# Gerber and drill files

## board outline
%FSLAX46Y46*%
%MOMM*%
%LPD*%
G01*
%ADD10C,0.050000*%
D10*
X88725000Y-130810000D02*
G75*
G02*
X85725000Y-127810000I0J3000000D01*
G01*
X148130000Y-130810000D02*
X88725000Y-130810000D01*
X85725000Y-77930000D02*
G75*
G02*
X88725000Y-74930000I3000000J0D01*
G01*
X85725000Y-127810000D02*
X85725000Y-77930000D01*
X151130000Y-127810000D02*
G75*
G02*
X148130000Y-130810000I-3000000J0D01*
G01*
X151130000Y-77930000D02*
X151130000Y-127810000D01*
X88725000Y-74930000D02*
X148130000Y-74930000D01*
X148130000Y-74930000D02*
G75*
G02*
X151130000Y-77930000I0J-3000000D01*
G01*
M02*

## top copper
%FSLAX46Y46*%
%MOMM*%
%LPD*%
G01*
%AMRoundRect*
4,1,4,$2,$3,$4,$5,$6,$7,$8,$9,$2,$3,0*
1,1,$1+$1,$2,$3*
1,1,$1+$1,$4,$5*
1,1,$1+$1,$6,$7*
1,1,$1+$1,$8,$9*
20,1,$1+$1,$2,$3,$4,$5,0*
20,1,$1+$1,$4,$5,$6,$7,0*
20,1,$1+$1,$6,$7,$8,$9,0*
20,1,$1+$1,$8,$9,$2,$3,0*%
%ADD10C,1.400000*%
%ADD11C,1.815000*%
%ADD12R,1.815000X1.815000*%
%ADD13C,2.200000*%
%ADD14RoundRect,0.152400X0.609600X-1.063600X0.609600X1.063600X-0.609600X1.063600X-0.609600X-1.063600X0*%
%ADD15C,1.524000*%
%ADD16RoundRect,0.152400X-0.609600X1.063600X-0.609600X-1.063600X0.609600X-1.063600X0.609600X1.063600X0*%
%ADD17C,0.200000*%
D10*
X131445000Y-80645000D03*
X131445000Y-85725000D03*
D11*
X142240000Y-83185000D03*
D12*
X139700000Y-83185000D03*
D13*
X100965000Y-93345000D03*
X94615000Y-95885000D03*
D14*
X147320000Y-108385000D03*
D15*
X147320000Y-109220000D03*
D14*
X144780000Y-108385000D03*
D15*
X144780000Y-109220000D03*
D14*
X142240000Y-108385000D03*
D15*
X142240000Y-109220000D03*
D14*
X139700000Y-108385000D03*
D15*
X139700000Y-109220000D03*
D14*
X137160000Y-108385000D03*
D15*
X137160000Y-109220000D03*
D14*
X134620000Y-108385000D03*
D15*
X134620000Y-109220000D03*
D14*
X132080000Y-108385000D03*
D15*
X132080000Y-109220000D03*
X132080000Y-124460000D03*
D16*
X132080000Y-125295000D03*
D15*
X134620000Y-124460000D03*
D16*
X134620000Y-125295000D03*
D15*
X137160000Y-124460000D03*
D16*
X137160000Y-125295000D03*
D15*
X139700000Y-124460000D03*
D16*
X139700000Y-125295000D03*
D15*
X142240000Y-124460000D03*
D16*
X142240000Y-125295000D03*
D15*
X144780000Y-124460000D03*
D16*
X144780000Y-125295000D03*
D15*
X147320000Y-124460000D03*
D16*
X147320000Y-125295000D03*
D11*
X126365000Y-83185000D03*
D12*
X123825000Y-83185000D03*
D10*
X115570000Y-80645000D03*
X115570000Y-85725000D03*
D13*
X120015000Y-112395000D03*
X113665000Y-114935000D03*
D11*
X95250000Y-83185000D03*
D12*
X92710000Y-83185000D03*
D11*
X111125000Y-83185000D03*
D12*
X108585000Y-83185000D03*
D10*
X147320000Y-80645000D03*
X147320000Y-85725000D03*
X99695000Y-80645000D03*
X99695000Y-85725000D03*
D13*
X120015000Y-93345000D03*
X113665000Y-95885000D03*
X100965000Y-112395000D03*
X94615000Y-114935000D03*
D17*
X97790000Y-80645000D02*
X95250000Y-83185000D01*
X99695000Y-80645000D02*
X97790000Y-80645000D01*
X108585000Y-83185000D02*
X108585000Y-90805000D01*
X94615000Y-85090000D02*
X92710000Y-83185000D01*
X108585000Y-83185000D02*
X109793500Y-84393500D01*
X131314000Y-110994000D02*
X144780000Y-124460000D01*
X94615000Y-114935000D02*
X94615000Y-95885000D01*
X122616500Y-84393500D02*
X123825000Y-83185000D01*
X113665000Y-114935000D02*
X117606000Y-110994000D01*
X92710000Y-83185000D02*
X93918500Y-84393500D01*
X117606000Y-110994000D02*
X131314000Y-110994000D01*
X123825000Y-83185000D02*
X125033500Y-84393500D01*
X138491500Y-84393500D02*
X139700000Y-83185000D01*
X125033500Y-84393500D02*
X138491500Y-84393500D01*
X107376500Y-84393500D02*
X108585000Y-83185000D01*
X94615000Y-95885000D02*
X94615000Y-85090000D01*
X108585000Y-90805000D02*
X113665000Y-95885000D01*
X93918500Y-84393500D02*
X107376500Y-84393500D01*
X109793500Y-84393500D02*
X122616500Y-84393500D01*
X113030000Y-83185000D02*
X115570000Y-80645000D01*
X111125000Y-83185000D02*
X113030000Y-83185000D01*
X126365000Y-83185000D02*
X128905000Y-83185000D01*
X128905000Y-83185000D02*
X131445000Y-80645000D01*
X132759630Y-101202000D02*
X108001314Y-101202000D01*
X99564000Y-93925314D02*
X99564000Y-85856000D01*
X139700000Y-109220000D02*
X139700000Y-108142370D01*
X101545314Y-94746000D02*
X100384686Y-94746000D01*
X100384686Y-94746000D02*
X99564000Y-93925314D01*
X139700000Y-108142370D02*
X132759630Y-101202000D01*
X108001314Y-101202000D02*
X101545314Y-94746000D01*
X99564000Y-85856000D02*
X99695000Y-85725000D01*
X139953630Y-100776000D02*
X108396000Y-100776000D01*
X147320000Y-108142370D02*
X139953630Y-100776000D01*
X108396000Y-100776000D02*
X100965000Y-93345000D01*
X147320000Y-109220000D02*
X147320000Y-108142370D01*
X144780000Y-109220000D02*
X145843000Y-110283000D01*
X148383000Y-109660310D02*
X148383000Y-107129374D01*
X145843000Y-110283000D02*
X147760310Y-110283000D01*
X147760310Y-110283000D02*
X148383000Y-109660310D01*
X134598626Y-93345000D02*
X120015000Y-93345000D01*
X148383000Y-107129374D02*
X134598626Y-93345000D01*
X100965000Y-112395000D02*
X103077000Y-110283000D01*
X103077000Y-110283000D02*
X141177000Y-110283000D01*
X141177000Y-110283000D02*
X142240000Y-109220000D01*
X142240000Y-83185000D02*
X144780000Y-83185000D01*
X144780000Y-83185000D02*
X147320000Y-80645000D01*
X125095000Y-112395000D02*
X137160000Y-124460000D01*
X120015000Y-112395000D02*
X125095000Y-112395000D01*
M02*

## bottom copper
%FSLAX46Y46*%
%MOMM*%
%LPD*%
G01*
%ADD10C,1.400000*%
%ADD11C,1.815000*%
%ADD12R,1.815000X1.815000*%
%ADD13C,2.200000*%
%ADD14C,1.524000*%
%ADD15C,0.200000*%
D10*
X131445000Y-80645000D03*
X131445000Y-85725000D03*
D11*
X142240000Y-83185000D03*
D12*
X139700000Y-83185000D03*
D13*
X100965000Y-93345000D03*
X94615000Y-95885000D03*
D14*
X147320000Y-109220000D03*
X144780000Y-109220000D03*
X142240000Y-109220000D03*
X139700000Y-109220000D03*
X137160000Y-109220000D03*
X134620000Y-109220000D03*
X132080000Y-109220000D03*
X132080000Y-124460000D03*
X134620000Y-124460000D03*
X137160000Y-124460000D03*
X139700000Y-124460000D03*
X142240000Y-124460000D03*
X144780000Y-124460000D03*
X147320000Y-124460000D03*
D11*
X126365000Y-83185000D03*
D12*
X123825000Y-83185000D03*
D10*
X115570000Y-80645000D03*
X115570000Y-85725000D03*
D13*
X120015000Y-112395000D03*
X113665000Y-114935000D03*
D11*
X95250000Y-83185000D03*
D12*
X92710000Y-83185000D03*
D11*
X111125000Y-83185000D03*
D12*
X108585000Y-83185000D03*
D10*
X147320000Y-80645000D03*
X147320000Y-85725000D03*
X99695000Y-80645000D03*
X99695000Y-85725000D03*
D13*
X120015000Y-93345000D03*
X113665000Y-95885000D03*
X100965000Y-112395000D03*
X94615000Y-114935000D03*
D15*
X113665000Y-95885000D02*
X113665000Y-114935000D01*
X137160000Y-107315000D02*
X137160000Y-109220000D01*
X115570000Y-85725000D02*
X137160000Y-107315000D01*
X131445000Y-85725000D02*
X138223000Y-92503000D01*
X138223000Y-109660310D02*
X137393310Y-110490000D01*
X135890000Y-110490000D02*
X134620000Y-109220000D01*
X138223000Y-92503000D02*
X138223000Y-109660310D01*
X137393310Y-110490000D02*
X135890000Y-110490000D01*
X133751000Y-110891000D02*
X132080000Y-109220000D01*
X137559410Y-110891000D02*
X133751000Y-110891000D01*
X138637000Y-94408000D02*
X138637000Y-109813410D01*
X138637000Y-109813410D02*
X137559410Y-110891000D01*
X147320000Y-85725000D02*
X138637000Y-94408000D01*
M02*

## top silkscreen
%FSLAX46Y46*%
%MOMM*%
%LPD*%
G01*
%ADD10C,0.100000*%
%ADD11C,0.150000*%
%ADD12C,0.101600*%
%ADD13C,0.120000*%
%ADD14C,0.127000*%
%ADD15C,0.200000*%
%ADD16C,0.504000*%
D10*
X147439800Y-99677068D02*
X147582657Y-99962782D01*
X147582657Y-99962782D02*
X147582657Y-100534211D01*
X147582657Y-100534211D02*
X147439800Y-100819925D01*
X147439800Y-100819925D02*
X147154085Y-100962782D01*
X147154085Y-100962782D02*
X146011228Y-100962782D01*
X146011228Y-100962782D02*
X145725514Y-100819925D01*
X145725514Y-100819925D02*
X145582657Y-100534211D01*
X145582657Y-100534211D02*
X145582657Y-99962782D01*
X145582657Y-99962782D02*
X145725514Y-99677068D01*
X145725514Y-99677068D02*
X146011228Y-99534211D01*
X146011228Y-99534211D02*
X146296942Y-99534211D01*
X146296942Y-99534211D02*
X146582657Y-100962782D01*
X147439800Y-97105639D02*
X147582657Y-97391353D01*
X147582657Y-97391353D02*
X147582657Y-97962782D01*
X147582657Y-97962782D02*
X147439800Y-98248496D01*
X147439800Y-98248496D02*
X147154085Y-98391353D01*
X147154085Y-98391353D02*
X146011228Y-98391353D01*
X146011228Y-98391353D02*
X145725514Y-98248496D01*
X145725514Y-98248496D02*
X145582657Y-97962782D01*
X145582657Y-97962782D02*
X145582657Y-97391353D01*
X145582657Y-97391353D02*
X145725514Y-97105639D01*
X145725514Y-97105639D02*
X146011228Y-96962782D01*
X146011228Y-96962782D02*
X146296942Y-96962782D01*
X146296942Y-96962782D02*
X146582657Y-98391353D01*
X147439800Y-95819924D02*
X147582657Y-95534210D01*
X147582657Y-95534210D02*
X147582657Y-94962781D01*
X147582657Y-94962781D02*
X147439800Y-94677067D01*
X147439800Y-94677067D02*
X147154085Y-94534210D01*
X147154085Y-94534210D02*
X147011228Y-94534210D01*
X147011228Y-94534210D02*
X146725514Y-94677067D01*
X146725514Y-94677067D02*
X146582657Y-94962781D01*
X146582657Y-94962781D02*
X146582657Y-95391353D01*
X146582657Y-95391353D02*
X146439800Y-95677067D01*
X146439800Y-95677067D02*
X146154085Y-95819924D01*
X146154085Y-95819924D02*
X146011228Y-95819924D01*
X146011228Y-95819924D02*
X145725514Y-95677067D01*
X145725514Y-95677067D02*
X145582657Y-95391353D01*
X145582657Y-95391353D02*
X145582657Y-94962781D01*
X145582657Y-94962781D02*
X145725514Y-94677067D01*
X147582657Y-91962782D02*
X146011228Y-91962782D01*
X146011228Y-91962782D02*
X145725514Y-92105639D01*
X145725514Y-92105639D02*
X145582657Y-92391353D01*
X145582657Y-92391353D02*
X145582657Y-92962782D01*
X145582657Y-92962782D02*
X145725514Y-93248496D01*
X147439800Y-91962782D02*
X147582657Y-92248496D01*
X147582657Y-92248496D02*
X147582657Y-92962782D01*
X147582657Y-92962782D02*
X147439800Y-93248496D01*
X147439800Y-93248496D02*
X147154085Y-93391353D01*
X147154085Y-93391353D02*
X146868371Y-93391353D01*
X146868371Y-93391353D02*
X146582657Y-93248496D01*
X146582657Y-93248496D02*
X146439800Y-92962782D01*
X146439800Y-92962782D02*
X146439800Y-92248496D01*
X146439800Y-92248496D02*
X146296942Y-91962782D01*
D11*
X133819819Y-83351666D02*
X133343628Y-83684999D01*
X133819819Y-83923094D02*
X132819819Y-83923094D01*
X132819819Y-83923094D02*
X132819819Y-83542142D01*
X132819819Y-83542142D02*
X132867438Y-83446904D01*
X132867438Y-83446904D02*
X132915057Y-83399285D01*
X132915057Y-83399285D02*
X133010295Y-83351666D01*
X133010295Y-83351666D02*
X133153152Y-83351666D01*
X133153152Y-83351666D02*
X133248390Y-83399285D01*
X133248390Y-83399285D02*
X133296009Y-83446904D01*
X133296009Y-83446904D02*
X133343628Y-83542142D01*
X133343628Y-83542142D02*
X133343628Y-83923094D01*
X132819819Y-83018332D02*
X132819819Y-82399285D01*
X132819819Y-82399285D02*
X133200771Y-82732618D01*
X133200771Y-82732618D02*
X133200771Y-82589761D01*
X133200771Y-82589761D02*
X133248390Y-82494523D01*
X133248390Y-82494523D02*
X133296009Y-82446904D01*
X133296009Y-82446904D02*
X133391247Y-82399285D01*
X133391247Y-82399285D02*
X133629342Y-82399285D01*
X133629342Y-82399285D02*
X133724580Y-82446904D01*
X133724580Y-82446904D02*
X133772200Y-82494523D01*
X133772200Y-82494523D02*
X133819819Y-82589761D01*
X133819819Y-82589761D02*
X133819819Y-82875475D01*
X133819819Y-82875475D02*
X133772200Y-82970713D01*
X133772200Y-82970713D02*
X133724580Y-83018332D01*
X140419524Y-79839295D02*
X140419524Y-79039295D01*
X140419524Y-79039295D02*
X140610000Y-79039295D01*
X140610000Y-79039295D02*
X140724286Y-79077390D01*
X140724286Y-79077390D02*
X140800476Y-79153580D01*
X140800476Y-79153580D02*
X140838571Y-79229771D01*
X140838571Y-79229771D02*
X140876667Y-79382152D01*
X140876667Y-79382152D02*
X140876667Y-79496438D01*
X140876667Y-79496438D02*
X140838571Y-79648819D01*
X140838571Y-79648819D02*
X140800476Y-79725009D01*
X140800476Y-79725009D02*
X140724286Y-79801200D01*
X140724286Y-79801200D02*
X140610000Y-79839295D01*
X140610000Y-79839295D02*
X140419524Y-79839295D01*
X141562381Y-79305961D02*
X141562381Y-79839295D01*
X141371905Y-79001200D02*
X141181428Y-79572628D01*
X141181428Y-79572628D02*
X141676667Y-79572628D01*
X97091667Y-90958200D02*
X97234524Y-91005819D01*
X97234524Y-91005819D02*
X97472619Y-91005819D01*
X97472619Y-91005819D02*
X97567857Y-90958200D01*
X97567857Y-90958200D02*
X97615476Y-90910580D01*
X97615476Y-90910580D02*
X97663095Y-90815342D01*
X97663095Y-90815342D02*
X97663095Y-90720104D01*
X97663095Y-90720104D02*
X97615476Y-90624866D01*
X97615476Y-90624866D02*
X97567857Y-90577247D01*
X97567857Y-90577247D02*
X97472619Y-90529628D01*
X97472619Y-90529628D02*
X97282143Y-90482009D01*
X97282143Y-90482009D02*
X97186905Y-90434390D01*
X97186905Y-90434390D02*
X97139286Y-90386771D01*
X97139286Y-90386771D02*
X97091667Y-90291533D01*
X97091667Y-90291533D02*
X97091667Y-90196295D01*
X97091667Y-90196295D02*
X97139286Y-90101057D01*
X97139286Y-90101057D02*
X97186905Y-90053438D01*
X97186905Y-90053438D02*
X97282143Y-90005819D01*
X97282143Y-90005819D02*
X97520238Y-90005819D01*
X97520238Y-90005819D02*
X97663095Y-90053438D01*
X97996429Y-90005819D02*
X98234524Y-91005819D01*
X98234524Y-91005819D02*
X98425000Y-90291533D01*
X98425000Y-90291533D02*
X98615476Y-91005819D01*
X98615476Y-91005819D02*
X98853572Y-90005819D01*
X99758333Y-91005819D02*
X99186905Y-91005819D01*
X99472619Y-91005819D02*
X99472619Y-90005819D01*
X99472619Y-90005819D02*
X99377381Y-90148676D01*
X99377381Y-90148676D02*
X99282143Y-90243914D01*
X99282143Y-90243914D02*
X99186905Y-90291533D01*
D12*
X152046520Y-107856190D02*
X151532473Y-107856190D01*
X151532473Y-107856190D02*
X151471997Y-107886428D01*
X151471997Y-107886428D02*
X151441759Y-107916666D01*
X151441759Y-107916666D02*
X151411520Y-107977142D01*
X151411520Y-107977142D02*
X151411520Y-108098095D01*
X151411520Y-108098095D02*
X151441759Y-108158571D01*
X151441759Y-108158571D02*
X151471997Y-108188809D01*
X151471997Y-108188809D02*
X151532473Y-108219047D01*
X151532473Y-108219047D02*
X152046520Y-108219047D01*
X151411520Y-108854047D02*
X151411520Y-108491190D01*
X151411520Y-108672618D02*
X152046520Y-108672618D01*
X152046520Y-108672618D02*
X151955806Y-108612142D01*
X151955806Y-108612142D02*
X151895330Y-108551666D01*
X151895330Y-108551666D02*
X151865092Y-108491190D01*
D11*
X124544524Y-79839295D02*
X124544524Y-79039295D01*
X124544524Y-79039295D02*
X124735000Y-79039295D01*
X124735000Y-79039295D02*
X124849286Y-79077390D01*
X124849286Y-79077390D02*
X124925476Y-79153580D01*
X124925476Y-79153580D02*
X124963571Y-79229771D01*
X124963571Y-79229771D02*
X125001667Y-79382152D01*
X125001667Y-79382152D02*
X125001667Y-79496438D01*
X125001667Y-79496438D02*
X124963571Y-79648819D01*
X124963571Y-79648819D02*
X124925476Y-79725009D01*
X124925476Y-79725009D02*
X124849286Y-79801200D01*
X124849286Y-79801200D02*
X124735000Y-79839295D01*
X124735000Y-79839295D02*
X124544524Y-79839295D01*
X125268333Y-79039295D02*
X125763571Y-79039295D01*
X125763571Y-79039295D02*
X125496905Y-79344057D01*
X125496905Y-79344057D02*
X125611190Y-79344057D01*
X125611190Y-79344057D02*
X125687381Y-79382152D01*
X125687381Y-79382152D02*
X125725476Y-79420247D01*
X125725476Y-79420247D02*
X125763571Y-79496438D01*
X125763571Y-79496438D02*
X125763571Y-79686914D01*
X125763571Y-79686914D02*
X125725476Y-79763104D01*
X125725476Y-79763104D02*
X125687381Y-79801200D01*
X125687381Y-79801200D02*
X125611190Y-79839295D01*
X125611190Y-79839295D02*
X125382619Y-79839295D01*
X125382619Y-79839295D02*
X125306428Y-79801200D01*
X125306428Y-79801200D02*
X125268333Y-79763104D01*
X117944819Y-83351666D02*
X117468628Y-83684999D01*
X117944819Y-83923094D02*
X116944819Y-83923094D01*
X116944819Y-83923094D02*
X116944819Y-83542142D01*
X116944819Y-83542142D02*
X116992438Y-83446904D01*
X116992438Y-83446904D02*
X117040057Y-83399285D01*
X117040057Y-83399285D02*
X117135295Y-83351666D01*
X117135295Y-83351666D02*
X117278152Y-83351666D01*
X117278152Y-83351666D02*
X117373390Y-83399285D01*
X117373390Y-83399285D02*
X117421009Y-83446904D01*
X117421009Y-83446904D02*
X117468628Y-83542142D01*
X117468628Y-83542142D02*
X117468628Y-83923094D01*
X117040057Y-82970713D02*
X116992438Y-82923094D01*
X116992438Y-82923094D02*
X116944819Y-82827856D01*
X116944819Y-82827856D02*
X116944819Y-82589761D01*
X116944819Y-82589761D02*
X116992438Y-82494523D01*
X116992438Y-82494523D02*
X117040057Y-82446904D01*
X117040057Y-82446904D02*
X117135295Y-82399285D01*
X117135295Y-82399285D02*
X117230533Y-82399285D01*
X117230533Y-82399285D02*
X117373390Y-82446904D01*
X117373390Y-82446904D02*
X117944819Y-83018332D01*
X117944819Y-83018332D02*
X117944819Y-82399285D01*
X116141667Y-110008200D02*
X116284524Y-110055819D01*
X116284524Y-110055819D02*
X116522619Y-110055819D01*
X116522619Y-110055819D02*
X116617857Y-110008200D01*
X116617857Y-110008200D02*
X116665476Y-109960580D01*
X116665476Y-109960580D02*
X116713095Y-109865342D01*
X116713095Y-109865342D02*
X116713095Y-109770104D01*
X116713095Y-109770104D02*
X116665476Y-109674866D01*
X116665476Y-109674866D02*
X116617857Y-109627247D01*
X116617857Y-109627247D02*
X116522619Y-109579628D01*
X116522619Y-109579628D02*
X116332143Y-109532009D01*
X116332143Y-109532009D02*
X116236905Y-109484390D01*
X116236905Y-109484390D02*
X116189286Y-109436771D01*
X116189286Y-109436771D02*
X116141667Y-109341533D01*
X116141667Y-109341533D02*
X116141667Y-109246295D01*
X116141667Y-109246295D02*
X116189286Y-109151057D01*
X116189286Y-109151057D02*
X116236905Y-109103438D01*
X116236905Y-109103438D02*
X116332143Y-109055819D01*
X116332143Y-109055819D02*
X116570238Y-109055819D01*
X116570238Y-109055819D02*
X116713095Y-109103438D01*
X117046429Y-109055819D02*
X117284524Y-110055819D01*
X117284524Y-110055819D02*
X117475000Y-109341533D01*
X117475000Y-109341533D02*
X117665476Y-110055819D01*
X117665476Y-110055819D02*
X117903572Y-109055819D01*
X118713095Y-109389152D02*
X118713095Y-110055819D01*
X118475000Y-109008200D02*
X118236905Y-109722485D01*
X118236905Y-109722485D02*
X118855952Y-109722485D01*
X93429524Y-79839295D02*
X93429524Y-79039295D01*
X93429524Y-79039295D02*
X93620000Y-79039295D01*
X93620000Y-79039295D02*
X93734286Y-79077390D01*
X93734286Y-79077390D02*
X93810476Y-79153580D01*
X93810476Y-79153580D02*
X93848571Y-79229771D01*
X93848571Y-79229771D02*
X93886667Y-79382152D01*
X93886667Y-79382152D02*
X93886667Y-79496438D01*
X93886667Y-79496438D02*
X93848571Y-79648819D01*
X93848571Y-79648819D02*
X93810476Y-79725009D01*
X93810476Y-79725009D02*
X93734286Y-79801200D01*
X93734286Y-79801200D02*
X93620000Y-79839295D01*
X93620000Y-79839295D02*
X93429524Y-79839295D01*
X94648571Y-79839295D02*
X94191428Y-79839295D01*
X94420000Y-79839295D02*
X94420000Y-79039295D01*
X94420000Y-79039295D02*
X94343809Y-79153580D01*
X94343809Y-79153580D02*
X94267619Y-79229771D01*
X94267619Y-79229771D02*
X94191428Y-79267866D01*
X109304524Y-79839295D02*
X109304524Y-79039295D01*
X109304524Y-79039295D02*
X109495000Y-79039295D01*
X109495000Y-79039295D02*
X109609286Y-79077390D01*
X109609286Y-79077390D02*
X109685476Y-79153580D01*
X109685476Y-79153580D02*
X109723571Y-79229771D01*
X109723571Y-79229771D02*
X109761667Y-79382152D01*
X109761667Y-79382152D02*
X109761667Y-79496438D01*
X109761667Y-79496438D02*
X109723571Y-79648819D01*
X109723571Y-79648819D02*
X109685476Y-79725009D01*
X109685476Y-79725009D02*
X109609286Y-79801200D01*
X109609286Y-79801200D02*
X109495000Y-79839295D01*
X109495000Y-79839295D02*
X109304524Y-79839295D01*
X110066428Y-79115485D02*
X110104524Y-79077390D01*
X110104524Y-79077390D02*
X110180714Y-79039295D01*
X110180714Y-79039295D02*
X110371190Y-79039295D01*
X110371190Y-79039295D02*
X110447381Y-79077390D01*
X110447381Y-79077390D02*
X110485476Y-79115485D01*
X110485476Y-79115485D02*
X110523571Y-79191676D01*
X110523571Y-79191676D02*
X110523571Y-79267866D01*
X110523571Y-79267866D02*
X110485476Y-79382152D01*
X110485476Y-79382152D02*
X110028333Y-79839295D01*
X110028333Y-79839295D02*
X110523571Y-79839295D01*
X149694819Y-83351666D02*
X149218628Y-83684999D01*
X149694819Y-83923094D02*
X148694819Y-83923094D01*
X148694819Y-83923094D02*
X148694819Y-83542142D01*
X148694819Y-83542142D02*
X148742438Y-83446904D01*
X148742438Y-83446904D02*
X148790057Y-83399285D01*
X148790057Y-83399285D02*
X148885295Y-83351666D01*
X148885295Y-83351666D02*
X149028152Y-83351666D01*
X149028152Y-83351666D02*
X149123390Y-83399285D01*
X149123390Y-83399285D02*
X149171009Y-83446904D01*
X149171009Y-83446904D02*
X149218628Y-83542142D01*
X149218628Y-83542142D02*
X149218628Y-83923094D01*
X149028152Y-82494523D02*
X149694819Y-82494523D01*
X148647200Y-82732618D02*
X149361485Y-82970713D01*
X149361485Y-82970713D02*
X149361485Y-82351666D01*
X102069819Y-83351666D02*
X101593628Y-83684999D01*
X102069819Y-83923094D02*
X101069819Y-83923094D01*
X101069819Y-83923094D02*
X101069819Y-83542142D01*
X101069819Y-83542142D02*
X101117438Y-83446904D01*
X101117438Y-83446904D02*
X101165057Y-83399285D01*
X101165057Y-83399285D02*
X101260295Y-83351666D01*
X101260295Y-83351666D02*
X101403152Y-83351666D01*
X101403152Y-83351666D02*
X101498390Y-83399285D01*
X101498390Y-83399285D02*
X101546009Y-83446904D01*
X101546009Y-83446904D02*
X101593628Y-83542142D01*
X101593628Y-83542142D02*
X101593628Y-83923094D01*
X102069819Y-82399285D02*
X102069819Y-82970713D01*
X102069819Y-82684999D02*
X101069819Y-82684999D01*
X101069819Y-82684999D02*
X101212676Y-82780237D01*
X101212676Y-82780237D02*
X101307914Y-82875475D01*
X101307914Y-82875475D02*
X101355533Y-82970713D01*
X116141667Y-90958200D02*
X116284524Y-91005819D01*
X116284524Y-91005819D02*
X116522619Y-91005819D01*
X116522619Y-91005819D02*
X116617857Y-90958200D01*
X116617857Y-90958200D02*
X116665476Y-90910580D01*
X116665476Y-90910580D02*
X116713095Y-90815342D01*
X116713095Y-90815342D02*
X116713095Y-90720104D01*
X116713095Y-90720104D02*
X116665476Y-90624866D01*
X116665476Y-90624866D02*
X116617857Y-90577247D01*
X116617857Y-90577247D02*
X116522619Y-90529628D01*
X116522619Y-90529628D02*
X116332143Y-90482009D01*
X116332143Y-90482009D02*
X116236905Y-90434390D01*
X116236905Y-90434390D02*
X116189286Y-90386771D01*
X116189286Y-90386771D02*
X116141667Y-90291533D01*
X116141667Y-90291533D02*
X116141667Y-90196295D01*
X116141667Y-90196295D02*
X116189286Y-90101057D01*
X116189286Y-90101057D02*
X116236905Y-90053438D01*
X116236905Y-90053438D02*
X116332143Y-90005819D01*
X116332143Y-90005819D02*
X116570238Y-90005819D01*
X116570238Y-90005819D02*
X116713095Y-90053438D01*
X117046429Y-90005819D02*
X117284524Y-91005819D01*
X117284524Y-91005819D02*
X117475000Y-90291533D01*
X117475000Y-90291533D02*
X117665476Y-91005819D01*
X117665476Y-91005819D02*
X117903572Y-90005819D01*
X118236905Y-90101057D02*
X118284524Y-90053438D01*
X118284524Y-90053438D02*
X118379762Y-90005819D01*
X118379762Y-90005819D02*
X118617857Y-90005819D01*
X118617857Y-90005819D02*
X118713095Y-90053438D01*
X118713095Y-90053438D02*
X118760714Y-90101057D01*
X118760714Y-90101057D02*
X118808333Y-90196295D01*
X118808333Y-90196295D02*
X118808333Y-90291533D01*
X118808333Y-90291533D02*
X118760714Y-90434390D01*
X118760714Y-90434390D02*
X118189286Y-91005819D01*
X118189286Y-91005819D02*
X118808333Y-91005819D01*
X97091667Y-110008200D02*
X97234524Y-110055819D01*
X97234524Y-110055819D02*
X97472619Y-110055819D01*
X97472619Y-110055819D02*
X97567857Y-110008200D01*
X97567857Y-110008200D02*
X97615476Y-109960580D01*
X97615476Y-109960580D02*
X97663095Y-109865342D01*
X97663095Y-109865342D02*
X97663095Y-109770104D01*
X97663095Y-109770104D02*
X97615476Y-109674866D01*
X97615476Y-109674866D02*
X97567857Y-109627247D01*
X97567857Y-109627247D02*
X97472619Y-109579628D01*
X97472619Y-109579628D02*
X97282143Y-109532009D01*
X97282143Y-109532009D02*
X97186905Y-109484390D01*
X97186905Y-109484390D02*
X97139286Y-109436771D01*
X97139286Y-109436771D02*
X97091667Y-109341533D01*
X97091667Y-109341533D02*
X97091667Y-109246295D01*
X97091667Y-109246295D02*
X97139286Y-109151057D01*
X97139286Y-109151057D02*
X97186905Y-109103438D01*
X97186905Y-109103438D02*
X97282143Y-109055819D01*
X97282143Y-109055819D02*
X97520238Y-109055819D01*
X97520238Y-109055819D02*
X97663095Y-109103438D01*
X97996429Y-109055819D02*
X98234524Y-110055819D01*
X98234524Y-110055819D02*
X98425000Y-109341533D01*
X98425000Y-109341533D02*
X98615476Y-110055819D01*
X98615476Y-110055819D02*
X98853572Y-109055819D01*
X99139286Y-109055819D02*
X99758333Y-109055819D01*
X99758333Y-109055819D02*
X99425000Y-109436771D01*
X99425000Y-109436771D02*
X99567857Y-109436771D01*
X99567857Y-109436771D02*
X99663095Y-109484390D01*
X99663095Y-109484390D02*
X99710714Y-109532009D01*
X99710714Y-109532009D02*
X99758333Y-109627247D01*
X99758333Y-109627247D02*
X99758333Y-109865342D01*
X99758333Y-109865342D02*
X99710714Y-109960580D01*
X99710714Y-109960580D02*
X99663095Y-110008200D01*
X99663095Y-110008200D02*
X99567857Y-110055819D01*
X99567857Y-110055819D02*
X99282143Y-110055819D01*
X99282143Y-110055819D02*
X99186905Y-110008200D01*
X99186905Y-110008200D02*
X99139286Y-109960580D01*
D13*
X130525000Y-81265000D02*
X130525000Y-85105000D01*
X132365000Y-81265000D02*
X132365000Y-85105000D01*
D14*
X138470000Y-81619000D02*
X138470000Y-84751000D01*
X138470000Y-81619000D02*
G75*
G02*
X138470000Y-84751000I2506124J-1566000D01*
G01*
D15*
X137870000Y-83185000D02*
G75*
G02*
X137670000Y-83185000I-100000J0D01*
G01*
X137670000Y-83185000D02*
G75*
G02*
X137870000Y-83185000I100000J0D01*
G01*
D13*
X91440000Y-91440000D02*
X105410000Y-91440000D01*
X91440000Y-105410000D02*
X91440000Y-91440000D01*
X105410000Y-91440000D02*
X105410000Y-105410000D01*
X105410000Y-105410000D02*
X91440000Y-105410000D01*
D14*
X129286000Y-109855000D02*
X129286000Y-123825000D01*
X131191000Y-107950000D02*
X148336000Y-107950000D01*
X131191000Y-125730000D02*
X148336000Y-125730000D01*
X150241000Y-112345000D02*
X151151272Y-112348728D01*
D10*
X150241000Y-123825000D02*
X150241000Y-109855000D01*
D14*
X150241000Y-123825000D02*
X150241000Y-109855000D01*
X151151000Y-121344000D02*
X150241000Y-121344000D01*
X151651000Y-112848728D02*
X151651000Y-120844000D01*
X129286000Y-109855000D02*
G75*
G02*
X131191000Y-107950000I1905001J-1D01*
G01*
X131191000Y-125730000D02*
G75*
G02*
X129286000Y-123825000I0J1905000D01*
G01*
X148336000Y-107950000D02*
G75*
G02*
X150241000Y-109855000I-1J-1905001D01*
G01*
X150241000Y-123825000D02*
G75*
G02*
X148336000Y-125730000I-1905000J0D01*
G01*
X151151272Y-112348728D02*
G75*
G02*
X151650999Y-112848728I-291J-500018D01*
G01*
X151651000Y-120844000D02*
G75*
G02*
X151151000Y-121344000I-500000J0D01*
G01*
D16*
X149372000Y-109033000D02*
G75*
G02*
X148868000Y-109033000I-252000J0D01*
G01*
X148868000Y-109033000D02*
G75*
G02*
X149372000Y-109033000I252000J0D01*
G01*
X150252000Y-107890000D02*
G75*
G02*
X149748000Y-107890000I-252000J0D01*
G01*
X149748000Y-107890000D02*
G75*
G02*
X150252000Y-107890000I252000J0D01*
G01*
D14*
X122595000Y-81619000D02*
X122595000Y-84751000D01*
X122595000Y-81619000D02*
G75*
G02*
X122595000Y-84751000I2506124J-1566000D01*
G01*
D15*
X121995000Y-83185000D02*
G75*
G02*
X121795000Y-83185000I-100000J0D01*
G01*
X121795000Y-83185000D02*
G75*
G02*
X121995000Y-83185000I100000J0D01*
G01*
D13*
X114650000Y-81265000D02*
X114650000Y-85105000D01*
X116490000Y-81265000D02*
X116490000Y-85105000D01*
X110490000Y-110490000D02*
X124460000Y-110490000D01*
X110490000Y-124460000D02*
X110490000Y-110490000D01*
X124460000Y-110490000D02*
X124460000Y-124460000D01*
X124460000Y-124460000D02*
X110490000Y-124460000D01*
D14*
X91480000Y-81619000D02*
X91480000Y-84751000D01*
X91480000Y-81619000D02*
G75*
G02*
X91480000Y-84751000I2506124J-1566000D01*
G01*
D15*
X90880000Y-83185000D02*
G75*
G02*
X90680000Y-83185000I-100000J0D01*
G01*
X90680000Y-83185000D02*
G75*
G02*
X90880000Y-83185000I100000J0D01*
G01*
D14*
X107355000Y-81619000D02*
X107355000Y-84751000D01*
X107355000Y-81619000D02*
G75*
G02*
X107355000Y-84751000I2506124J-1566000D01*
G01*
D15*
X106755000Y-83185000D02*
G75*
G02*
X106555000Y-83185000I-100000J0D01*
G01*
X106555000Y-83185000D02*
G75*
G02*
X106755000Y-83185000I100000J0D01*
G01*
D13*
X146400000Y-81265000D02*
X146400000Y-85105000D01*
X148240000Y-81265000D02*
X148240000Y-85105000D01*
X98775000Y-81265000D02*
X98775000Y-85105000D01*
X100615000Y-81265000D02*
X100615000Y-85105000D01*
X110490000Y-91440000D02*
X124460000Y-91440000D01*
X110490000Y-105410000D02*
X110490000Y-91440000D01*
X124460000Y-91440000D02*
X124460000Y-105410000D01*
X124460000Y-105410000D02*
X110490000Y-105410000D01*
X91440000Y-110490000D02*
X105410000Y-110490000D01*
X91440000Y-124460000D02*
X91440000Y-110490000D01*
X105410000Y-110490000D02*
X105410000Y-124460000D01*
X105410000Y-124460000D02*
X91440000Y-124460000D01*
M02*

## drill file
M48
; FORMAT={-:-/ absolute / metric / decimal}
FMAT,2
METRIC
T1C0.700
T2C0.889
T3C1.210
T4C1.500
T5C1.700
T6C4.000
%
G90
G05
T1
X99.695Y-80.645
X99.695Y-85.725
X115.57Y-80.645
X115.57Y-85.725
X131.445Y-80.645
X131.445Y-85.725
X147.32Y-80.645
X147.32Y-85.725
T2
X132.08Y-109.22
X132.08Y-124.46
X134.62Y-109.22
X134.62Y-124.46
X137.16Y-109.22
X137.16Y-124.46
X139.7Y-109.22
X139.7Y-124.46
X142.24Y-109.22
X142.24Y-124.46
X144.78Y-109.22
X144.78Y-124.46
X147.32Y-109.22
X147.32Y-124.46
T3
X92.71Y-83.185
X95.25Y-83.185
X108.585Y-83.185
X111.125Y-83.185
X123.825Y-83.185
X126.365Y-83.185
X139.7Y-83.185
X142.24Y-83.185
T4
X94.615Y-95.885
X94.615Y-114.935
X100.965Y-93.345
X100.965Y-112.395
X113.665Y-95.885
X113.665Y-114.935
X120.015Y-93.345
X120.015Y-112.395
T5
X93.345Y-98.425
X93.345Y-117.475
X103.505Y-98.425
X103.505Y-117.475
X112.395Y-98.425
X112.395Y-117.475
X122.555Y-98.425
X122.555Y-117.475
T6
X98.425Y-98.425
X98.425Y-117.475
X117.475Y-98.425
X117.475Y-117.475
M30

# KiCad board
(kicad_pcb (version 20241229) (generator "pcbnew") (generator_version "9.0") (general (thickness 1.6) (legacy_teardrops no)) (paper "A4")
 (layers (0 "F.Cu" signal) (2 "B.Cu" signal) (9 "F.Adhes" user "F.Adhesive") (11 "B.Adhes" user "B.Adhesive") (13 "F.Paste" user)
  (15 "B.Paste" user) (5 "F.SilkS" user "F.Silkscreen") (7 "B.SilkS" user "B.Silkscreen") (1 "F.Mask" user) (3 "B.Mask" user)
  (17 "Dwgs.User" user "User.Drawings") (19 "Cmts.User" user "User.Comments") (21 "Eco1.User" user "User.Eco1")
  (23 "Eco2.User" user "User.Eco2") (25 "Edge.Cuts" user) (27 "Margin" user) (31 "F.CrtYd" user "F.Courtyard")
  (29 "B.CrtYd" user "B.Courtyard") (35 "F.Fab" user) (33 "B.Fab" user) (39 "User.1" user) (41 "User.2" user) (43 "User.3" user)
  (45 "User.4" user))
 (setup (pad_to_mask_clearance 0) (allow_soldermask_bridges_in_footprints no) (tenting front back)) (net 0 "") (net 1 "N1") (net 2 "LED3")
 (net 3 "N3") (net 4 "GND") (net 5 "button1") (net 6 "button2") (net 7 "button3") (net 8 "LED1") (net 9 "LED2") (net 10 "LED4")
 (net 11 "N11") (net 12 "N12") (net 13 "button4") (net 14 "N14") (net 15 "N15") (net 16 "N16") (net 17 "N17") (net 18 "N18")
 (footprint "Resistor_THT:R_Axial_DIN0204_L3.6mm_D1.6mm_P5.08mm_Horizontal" (layer "F.Cu") (at 131.445 80.645 -90)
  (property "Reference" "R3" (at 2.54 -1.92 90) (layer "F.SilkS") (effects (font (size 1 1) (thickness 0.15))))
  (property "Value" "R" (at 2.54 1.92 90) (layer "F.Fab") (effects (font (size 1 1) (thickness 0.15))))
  (fp_line (start 0.62 0.92) (end 4.46 0.92) (stroke (width 0.12) (type solid)) (layer "F.SilkS"))
  (fp_line (start 0.62 -0.92) (end 4.46 -0.92) (stroke (width 0.12) (type solid)) (layer "F.SilkS"))
  (pad "1" thru_hole circle (at 0 0 270) (size 1.4 1.4) (drill 0.7) (layers "*.Cu" "*.Mask") (remove_unused_layers no) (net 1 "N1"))
  (pad "2" thru_hole circle (at 5.08 0 270) (size 1.4 1.4) (drill 0.7) (layers "*.Cu" "*.Mask") (remove_unused_layers no) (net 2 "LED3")))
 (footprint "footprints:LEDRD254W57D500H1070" (layer "F.Cu") (at 140.97 83.185)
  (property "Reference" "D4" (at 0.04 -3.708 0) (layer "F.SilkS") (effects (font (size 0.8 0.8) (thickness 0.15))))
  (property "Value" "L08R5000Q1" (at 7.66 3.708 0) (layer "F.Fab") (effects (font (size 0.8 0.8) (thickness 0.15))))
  (fp_line (start -2.5 -1.566) (end -2.5 1.566) (stroke (width 0.127) (type solid)) (layer "F.SilkS"))
  (fp_arc (start -2.5 -1.566) (mid 2.961291 0) (end -2.5 1.566) (stroke (width 0.127) (type solid)) (layer "F.SilkS"))
  (fp_circle (center -3.2 0) (end -3.1 0) (stroke (width 0.2) (type solid)) (fill no) (layer "F.SilkS"))
  (pad "A" thru_hole circle (at 1.27 0) (size 1.815 1.815) (drill 1.21) (layers "*.Cu" "*.Mask") (remove_unused_layers no) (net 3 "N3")
   (solder_mask_margin 0.102))
  (pad "C" thru_hole rect (at -1.27 0) (size 1.815 1.815) (drill 1.21) (layers "*.Cu" "*.Mask") (remove_unused_layers no) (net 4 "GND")
   (solder_mask_margin 0.102)))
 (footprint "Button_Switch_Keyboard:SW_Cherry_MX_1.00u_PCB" (layer "F.Cu") (at 100.965 93.345)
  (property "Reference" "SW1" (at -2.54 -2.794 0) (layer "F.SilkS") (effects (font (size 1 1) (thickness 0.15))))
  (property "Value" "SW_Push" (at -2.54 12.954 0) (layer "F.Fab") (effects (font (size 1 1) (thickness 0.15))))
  (fp_line (start -9.525 -1.905) (end 4.445 -1.905) (stroke (width 0.12) (type solid)) (layer "F.SilkS"))
  (fp_line (start -9.525 12.065) (end -9.525 -1.905) (stroke (width 0.12) (type solid)) (layer "F.SilkS"))
  (fp_line (start 4.445 -1.905) (end 4.445 12.065) (stroke (width 0.12) (type solid)) (layer "F.SilkS"))
  (fp_line (start 4.445 12.065) (end -9.525 12.065) (stroke (width 0.12) (type solid)) (layer "F.SilkS"))
  (pad "" np_thru_hole circle (at -7.62 5.08) (size 1.7 1.7) (drill 1.7) (layers "*.Cu" "*.Mask"))
  (pad "" np_thru_hole circle (at -2.54 5.08) (size 4 4) (drill 4) (layers "*.Cu" "*.Mask"))
  (pad "" np_thru_hole circle (at 2.54 5.08) (size 1.7 1.7) (drill 1.7) (layers "*.Cu" "*.Mask"))
  (pad "1" thru_hole circle (at 0 0) (size 2.2 2.2) (drill 1.5) (layers "*.Cu" "*.Mask") (remove_unused_layers no) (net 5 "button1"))
  (pad "2" thru_hole circle (at -6.35 2.54) (size 2.2 2.2) (drill 1.5) (layers "*.Cu" "*.Mask") (remove_unused_layers no) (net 4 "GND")))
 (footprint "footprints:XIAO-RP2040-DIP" (layer "F.Cu") (at 139.7 116.84 -90)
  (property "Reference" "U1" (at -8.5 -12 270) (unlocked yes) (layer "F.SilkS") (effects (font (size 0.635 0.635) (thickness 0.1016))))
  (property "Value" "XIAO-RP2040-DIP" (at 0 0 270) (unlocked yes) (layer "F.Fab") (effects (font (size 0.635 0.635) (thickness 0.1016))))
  (fp_line (start -6.985 10.414) (end 6.985 10.414) (stroke (width 0.127) (type solid)) (layer "F.SilkS"))
  (fp_line (start -8.89 8.509) (end -8.89 -8.636) (stroke (width 0.127) (type solid)) (layer "F.SilkS"))
  (fp_line (start 8.89 8.509) (end 8.89 -8.636) (stroke (width 0.127) (type solid)) (layer "F.SilkS"))
  (fp_line (start -4.495 -10.541) (end -4.491272 -11.451272) (stroke (width 0.127) (type solid)) (layer "F.SilkS"))
  (fp_line (start 6.985 -10.541) (end -6.985 -10.541) (stroke (width 0.1) (type solid)) (layer "F.SilkS"))
  (fp_line (start 6.985 -10.541) (end -6.985 -10.541) (stroke (width 0.127) (type solid)) (layer "F.SilkS"))
  (fp_line (start 4.504 -11.451) (end 4.504 -10.541) (stroke (width 0.127) (type solid)) (layer "F.SilkS"))
  (fp_line (start -3.991272 -11.951) (end 4.004 -11.951) (stroke (width 0.127) (type solid)) (layer "F.SilkS"))
  (fp_arc (start -6.985 10.414) (mid -8.332038 9.856038) (end -8.89 8.509) (stroke (width 0.127) (type solid)) (layer "F.SilkS"))
  (fp_arc (start 8.89 8.509) (mid 8.332038 9.856038) (end 6.985 10.414) (stroke (width 0.127) (type solid)) (layer "F.SilkS"))
  (fp_arc (start -8.89 -8.636) (mid -8.332038 -9.983038) (end -6.985 -10.541) (stroke (width 0.127) (type solid)) (layer "F.SilkS"))
  (fp_arc (start 6.985 -10.541) (mid 8.332038 -9.983038) (end 8.89 -8.636) (stroke (width 0.127) (type solid)) (layer "F.SilkS"))
  (fp_arc (start -4.491272 -11.451272) (mid -4.344728 -11.80464) (end -3.991272 -11.951) (stroke (width 0.127) (type default))
   (layer "F.SilkS"))
  (fp_arc (start 4.004 -11.951) (mid 4.357553 -11.804553) (end 4.504 -11.451) (stroke (width 0.127) (type default)) (layer "F.SilkS"))
  (fp_circle (center -7.807 -9.42) (end -7.807 -9.674) (stroke (width 0.5) (type solid)) (fill yes) (layer "F.SilkS"))
  (fp_circle (center -8.95 -10.3) (end -8.95 -10.554) (stroke (width 0.5) (type solid)) (fill yes) (layer "F.SilkS"))
  (pad "1" smd roundrect (at -8.455 -7.62 90) (size 2.432 1.524) (layers "F.Cu" "F.Mask") (roundrect_rratio 0.1) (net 5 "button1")
   (thermal_bridge_angle 45))
  (pad "1" thru_hole circle (at -7.62 -7.62 90) (size 1.524 1.524) (drill 0.889) (layers "*.Cu" "*.Mask") (remove_unused_layers no)
   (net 5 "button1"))
  (pad "2" smd roundrect (at -8.455 -5.08 90) (size 2.432 1.524) (layers "F.Cu" "F.Mask") (roundrect_rratio 0.1) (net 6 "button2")
   (thermal_bridge_angle 45))
  (pad "2" thru_hole circle (at -7.62 -5.08 90) (size 1.524 1.524) (drill 0.889) (layers "*.Cu" "*.Mask") (remove_unused_layers no)
   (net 6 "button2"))
  (pad "3" smd roundrect (at -8.455 -2.54 90) (size 2.432 1.524) (layers "F.Cu" "F.Mask") (roundrect_rratio 0.1) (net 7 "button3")
   (thermal_bridge_angle 45))
  (pad "3" thru_hole circle (at -7.62 -2.54 90) (size 1.524 1.524) (drill 0.889) (layers "*.Cu" "*.Mask") (remove_unused_layers no)
   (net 7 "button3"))
  (pad "4" smd roundrect (at -8.455 0 90) (size 2.432 1.524) (layers "F.Cu" "F.Mask") (roundrect_rratio 0.1) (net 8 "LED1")
   (thermal_bridge_angle 45))
  (pad "4" thru_hole circle (at -7.62 0 90) (size 1.524 1.524) (drill 0.889) (layers "*.Cu" "*.Mask") (remove_unused_layers no)
   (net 8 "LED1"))
  (pad "5" smd roundrect (at -8.455 2.54 90) (size 2.432 1.524) (layers "F.Cu" "F.Mask") (roundrect_rratio 0.1) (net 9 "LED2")
   (thermal_bridge_angle 45))
  (pad "5" thru_hole circle (at -7.62 2.54 90) (size 1.524 1.524) (drill 0.889) (layers "*.Cu" "*.Mask") (remove_unused_layers no)
   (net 9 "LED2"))
  (pad "6" smd roundrect (at -8.455 5.08 90) (size 2.432 1.524) (layers "F.Cu" "F.Mask") (roundrect_rratio 0.1) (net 2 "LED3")
   (thermal_bridge_angle 45))
  (pad "6" thru_hole circle (at -7.62 5.08 90) (size 1.524 1.524) (drill 0.889) (layers "*.Cu" "*.Mask") (remove_unused_layers no)
   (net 2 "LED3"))
  (pad "7" smd roundrect (at -8.455 7.62 90) (size 2.432 1.524) (layers "F.Cu" "F.Mask") (roundrect_rratio 0.1) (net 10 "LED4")
   (thermal_bridge_angle 45))
  (pad "7" thru_hole circle (at -7.62 7.62 90) (size 1.524 1.524) (drill 0.889) (layers "*.Cu" "*.Mask") (remove_unused_layers no)
   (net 10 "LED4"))
  (pad "8" thru_hole circle (at 7.62 7.62 270) (size 1.524 1.524) (drill 0.889) (layers "*.Cu" "*.Mask") (remove_unused_layers no)
   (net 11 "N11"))
  (pad "8" smd roundrect (at 8.455 7.62 270) (size 2.432 1.524) (layers "F.Cu" "F.Mask") (roundrect_rratio 0.1) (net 11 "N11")
   (thermal_bridge_angle 45))
  (pad "9" thru_hole circle (at 7.62 5.08 270) (size 1.524 1.524) (drill 0.889) (layers "*.Cu" "*.Mask") (remove_unused_layers no)
   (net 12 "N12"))
  (pad "9" smd roundrect (at 8.455 5.08 270) (size 2.432 1.524) (layers "F.Cu" "F.Mask") (roundrect_rratio 0.1) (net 12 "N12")
   (thermal_bridge_angle 45))
  (pad "10" thru_hole circle (at 7.62 2.54 270) (size 1.524 1.524) (drill 0.889) (layers "*.Cu" "*.Mask") (remove_unused_layers no)
   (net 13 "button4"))
  (pad "10" smd roundrect (at 8.455 2.54 270) (size 2.432 1.524) (layers "F.Cu" "F.Mask") (roundrect_rratio 0.1) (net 13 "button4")
   (thermal_bridge_angle 45))
  (pad "11" thru_hole circle (at 7.62 0 270) (size 1.524 1.524) (drill 0.889) (layers "*.Cu" "*.Mask") (remove_unused_layers no)
   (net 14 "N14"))
  (pad "11" smd roundrect (at 8.455 0 270) (size 2.432 1.524) (layers "F.Cu" "F.Mask") (roundrect_rratio 0.1) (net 14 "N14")
   (thermal_bridge_angle 45))
  (pad "12" thru_hole circle (at 7.62 -2.54 270) (size 1.524 1.524) (drill 0.889) (layers "*.Cu" "*.Mask") (remove_unused_layers no)
   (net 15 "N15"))
  (pad "12" smd roundrect (at 8.455 -2.54 270) (size 2.432 1.524) (layers "F.Cu" "F.Mask") (roundrect_rratio 0.1) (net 15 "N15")
   (thermal_bridge_angle 45))
  (pad "13" thru_hole circle (at 7.62 -5.08 270) (size 1.524 1.524) (drill 0.889) (layers "*.Cu" "*.Mask") (remove_unused_layers no)
   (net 4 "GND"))
  (pad "13" smd roundrect (at 8.455 -5.08 270) (size 2.432 1.524) (layers "F.Cu" "F.Mask") (roundrect_rratio 0.1) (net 4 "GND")
   (thermal_bridge_angle 45))
  (pad "14" thru_hole circle (at 7.62 -7.62 270) (size 1.524 1.524) (drill 0.889) (layers "*.Cu" "*.Mask") (remove_unused_layers no)
   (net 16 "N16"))
  (pad "14" smd roundrect (at 8.455 -7.62 270) (size 2.432 1.524) (layers "F.Cu" "F.Mask") (roundrect_rratio 0.1) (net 16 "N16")
   (thermal_bridge_angle 45)))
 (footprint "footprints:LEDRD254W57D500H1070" (layer "F.Cu") (at 125.095 83.185)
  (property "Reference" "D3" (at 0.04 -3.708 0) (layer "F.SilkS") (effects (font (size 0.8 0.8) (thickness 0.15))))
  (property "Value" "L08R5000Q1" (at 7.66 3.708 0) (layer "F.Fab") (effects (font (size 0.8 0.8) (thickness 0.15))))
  (fp_line (start -2.5 -1.566) (end -2.5 1.566) (stroke (width 0.127) (type solid)) (layer "F.SilkS"))
  (fp_arc (start -2.5 -1.566) (mid 2.961291 0) (end -2.5 1.566) (stroke (width 0.127) (type solid)) (layer "F.SilkS"))
  (fp_circle (center -3.2 0) (end -3.1 0) (stroke (width 0.2) (type solid)) (fill no) (layer "F.SilkS"))
  (pad "A" thru_hole circle (at 1.27 0) (size 1.815 1.815) (drill 1.21) (layers "*.Cu" "*.Mask") (remove_unused_layers no) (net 1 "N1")
   (solder_mask_margin 0.102))
  (pad "C" thru_hole rect (at -1.27 0) (size 1.815 1.815) (drill 1.21) (layers "*.Cu" "*.Mask") (remove_unused_layers no) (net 4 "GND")
   (solder_mask_margin 0.102)))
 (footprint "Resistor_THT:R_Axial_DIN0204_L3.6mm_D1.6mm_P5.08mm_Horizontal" (layer "F.Cu") (at 115.57 80.645 -90)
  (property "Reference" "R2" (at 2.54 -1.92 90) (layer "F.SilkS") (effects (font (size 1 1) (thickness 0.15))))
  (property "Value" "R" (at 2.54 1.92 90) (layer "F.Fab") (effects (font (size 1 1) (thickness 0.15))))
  (fp_line (start 0.62 0.92) (end 4.46 0.92) (stroke (width 0.12) (type solid)) (layer "F.SilkS"))
  (fp_line (start 0.62 -0.92) (end 4.46 -0.92) (stroke (width 0.12) (type solid)) (layer "F.SilkS"))
  (pad "1" thru_hole circle (at 0 0 270) (size 1.4 1.4) (drill 0.7) (layers "*.Cu" "*.Mask") (remove_unused_layers no) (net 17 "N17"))
  (pad "2" thru_hole circle (at 5.08 0 270) (size 1.4 1.4) (drill 0.7) (layers "*.Cu" "*.Mask") (remove_unused_layers no) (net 9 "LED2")))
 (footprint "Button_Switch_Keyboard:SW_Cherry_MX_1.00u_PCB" (layer "F.Cu") (at 120.015 112.395)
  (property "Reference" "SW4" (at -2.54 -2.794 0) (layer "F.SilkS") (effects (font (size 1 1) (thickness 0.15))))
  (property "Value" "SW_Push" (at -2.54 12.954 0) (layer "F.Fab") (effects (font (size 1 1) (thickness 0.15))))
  (fp_line (start -9.525 -1.905) (end 4.445 -1.905) (stroke (width 0.12) (type solid)) (layer "F.SilkS"))
  (fp_line (start -9.525 12.065) (end -9.525 -1.905) (stroke (width 0.12) (type solid)) (layer "F.SilkS"))
  (fp_line (start 4.445 -1.905) (end 4.445 12.065) (stroke (width 0.12) (type solid)) (layer "F.SilkS"))
  (fp_line (start 4.445 12.065) (end -9.525 12.065) (stroke (width 0.12) (type solid)) (layer "F.SilkS"))
  (pad "" np_thru_hole circle (at -7.62 5.08) (size 1.7 1.7) (drill 1.7) (layers "*.Cu" "*.Mask"))
  (pad "" np_thru_hole circle (at -2.54 5.08) (size 4 4) (drill 4) (layers "*.Cu" "*.Mask"))
  (pad "" np_thru_hole circle (at 2.54 5.08) (size 1.7 1.7) (drill 1.7) (layers "*.Cu" "*.Mask"))
  (pad "1" thru_hole circle (at 0 0) (size 2.2 2.2) (drill 1.5) (layers "*.Cu" "*.Mask") (remove_unused_layers no) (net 13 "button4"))
  (pad "2" thru_hole circle (at -6.35 2.54) (size 2.2 2.2) (drill 1.5) (layers "*.Cu" "*.Mask") (remove_unused_layers no) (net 4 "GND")))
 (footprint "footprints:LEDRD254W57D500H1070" (layer "F.Cu") (at 93.98 83.185)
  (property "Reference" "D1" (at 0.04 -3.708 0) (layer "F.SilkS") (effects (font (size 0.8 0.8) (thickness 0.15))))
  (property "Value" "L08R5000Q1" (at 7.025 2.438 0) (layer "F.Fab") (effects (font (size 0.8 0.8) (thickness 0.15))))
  (fp_line (start -2.5 -1.566) (end -2.5 1.566) (stroke (width 0.127) (type solid)) (layer "F.SilkS"))
  (fp_arc (start -2.5 -1.566) (mid 2.961291 0) (end -2.5 1.566) (stroke (width 0.127) (type solid)) (layer "F.SilkS"))
  (fp_circle (center -3.2 0) (end -3.1 0) (stroke (width 0.2) (type solid)) (fill no) (layer "F.SilkS"))
  (pad "A" thru_hole circle (at 1.27 0) (size 1.815 1.815) (drill 1.21) (layers "*.Cu" "*.Mask") (remove_unused_layers no) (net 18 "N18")
   (solder_mask_margin 0.102))
  (pad "C" thru_hole rect (at -1.27 0) (size 1.815 1.815) (drill 1.21) (layers "*.Cu" "*.Mask") (remove_unused_layers no) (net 4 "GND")
   (solder_mask_margin 0.102)))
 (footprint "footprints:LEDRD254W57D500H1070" (layer "F.Cu") (at 109.855 83.185)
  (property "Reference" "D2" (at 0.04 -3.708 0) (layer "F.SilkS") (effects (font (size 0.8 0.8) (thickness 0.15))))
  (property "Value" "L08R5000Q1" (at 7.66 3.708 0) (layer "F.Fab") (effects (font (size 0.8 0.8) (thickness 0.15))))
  (fp_line (start -2.5 -1.566) (end -2.5 1.566) (stroke (width 0.127) (type solid)) (layer "F.SilkS"))
  (fp_arc (start -2.5 -1.566) (mid 2.961291 0) (end -2.5 1.566) (stroke (width 0.127) (type solid)) (layer "F.SilkS"))
  (fp_circle (center -3.2 0) (end -3.1 0) (stroke (width 0.2) (type solid)) (fill no) (layer "F.SilkS"))
  (pad "A" thru_hole circle (at 1.27 0) (size 1.815 1.815) (drill 1.21) (layers "*.Cu" "*.Mask") (remove_unused_layers no) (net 17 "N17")
   (solder_mask_margin 0.102))
  (pad "C" thru_hole rect (at -1.27 0) (size 1.815 1.815) (drill 1.21) (layers "*.Cu" "*.Mask") (remove_unused_layers no) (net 4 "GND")
   (solder_mask_margin 0.102)))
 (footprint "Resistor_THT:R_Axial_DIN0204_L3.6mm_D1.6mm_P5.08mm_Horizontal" (layer "F.Cu") (at 147.32 80.645 -90)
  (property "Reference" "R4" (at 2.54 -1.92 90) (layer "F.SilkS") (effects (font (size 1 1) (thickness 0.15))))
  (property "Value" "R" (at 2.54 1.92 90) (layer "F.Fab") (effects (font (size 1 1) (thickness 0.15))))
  (fp_line (start 0.62 0.92) (end 4.46 0.92) (stroke (width 0.12) (type solid)) (layer "F.SilkS"))
  (fp_line (start 0.62 -0.92) (end 4.46 -0.92) (stroke (width 0.12) (type solid)) (layer "F.SilkS"))
  (pad "1" thru_hole circle (at 0 0 270) (size 1.4 1.4) (drill 0.7) (layers "*.Cu" "*.Mask") (remove_unused_layers no) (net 3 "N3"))
  (pad "2" thru_hole circle (at 5.08 0 270) (size 1.4 1.4) (drill 0.7) (layers "*.Cu" "*.Mask") (remove_unused_layers no) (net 10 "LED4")))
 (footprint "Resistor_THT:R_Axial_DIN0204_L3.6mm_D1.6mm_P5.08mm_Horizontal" (layer "F.Cu") (at 99.695 80.645 -90)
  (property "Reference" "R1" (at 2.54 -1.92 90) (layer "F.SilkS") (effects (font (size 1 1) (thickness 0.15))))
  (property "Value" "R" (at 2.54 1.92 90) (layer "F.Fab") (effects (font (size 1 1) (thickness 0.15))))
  (fp_line (start 0.62 0.92) (end 4.46 0.92) (stroke (width 0.12) (type solid)) (layer "F.SilkS"))
  (fp_line (start 0.62 -0.92) (end 4.46 -0.92) (stroke (width 0.12) (type solid)) (layer "F.SilkS"))
  (pad "1" thru_hole circle (at 0 0 270) (size 1.4 1.4) (drill 0.7) (layers "*.Cu" "*.Mask") (remove_unused_layers no) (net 18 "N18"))
  (pad "2" thru_hole circle (at 5.08 0 270) (size 1.4 1.4) (drill 0.7) (layers "*.Cu" "*.Mask") (remove_unused_layers no) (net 8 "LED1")))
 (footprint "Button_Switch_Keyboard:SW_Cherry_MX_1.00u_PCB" (layer "F.Cu") (at 120.015 93.345)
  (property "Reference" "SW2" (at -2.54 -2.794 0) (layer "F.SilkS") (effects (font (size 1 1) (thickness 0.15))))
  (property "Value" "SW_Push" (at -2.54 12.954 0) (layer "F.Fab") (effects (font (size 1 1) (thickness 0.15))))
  (fp_line (start -9.525 -1.905) (end 4.445 -1.905) (stroke (width 0.12) (type solid)) (layer "F.SilkS"))
  (fp_line (start -9.525 12.065) (end -9.525 -1.905) (stroke (width 0.12) (type solid)) (layer "F.SilkS"))
  (fp_line (start 4.445 -1.905) (end 4.445 12.065) (stroke (width 0.12) (type solid)) (layer "F.SilkS"))
  (fp_line (start 4.445 12.065) (end -9.525 12.065) (stroke (width 0.12) (type solid)) (layer "F.SilkS"))
  (pad "" np_thru_hole circle (at -7.62 5.08) (size 1.7 1.7) (drill 1.7) (layers "*.Cu" "*.Mask"))
  (pad "" np_thru_hole circle (at -2.54 5.08) (size 4 4) (drill 4) (layers "*.Cu" "*.Mask"))
  (pad "" np_thru_hole circle (at 2.54 5.08) (size 1.7 1.7) (drill 1.7) (layers "*.Cu" "*.Mask"))
  (pad "1" thru_hole circle (at 0 0) (size 2.2 2.2) (drill 1.5) (layers "*.Cu" "*.Mask") (remove_unused_layers no) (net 6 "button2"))
  (pad "2" thru_hole circle (at -6.35 2.54) (size 2.2 2.2) (drill 1.5) (layers "*.Cu" "*.Mask") (remove_unused_layers no) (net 4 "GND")))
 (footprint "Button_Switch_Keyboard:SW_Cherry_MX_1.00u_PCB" (layer "F.Cu") (at 100.965 112.395)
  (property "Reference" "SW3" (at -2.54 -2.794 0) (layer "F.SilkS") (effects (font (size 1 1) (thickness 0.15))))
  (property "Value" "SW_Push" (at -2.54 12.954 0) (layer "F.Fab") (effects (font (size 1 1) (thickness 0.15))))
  (fp_line (start -9.525 -1.905) (end 4.445 -1.905) (stroke (width 0.12) (type solid)) (layer "F.SilkS"))
  (fp_line (start -9.525 12.065) (end -9.525 -1.905) (stroke (width 0.12) (type solid)) (layer "F.SilkS"))
  (fp_line (start 4.445 -1.905) (end 4.445 12.065) (stroke (width 0.12) (type solid)) (layer "F.SilkS"))
  (fp_line (start 4.445 12.065) (end -9.525 12.065) (stroke (width 0.12) (type solid)) (layer "F.SilkS"))
  (pad "" np_thru_hole circle (at -7.62 5.08) (size 1.7 1.7) (drill 1.7) (layers "*.Cu" "*.Mask"))
  (pad "" np_thru_hole circle (at -2.54 5.08) (size 4 4) (drill 4) (layers "*.Cu" "*.Mask"))
  (pad "" np_thru_hole circle (at 2.54 5.08) (size 1.7 1.7) (drill 1.7) (layers "*.Cu" "*.Mask"))
  (pad "1" thru_hole circle (at 0 0) (size 2.2 2.2) (drill 1.5) (layers "*.Cu" "*.Mask") (remove_unused_layers no) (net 7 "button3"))
  (pad "2" thru_hole circle (at -6.35 2.54) (size 2.2 2.2) (drill 1.5) (layers "*.Cu" "*.Mask") (remove_unused_layers no) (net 4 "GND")))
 (gr_arc (start 88.725 130.81) (mid 86.60368 129.93132) (end 85.725 127.81) (stroke (width 0.05) (type default)) (layer "Edge.Cuts"))
 (gr_line (start 148.13 130.81) (end 88.725 130.81) (stroke (width 0.05) (type default)) (layer "Edge.Cuts"))
 (gr_arc (start 85.725 77.93) (mid 86.60368 75.80868) (end 88.725 74.93) (stroke (width 0.05) (type default)) (layer "Edge.Cuts"))
 (gr_line (start 85.725 127.81) (end 85.725 77.93) (stroke (width 0.05) (type default)) (layer "Edge.Cuts"))
 (gr_arc (start 151.13 127.81) (mid 150.25132 129.93132) (end 148.13 130.81) (stroke (width 0.05) (type default)) (layer "Edge.Cuts"))
 (gr_line (start 151.13 77.93) (end 151.13 127.81) (stroke (width 0.05) (type default)) (layer "Edge.Cuts"))
 (gr_line (start 88.725 74.93) (end 148.13 74.93) (stroke (width 0.05) (type default)) (layer "Edge.Cuts"))
 (gr_arc (start 148.13 74.93) (mid 150.25132 75.80868) (end 151.13 77.93) (stroke (width 0.05) (type default)) (layer "Edge.Cuts"))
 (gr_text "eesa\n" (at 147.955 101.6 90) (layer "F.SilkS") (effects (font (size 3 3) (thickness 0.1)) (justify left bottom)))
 (segment (start 97.79 80.645) (end 95.25 83.185) (width 0.2) (layer "F.Cu") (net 18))
 (segment (start 99.695 80.645) (end 97.79 80.645) (width 0.2) (layer "F.Cu") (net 18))
 (segment (start 108.585 83.185) (end 108.585 90.805) (width 0.2) (layer "F.Cu") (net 4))
 (segment (start 94.615 85.09) (end 92.71 83.185) (width 0.2) (layer "F.Cu") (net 4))
 (segment (start 108.585 83.185) (end 109.7935 84.3935) (width 0.2) (layer "F.Cu") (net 4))
 (segment (start 131.314 110.994) (end 144.78 124.46) (width 0.2) (layer "F.Cu") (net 4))
 (segment (start 94.615 114.935) (end 94.615 95.885) (width 0.2) (layer "F.Cu") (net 4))
 (segment (start 122.6165 84.3935) (end 123.825 83.185) (width 0.2) (layer "F.Cu") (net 4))
 (segment (start 113.665 114.935) (end 117.606 110.994) (width 0.2) (layer "F.Cu") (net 4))
 (segment (start 92.71 83.185) (end 93.9185 84.3935) (width 0.2) (layer "F.Cu") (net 4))
 (segment (start 117.606 110.994) (end 131.314 110.994) (width 0.2) (layer "F.Cu") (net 4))
 (segment (start 123.825 83.185) (end 125.0335 84.3935) (width 0.2) (layer "F.Cu") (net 4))
 (segment (start 138.4915 84.3935) (end 139.7 83.185) (width 0.2) (layer "F.Cu") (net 4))
 (segment (start 125.0335 84.3935) (end 138.4915 84.3935) (width 0.2) (layer "F.Cu") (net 4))
 (segment (start 107.3765 84.3935) (end 108.585 83.185) (width 0.2) (layer "F.Cu") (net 4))
 (segment (start 94.615 95.885) (end 94.615 85.09) (width 0.2) (layer "F.Cu") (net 4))
 (segment (start 108.585 90.805) (end 113.665 95.885) (width 0.2) (layer "F.Cu") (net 4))
 (segment (start 93.9185 84.3935) (end 107.3765 84.3935) (width 0.2) (layer "F.Cu") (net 4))
 (segment (start 109.7935 84.3935) (end 122.6165 84.3935) (width 0.2) (layer "F.Cu") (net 4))
 (segment (start 113.665 95.885) (end 113.665 114.935) (width 0.2) (layer "B.Cu") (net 4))
 (segment (start 113.03 83.185) (end 115.57 80.645) (width 0.2) (layer "F.Cu") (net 17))
 (segment (start 111.125 83.185) (end 113.03 83.185) (width 0.2) (layer "F.Cu") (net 17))
 (segment (start 126.365 83.185) (end 128.905 83.185) (width 0.2) (layer "F.Cu") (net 1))
 (segment (start 128.905 83.185) (end 131.445 80.645) (width 0.2) (layer "F.Cu") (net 1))
 (segment (start 132.75963 101.202) (end 108.001314 101.202) (width 0.2) (layer "F.Cu") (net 8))
 (segment (start 99.564 93.925314) (end 99.564 85.856) (width 0.2) (layer "F.Cu") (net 8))
 (segment (start 139.7 109.22) (end 139.7 108.14237) (width 0.2) (layer "F.Cu") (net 8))
 (segment (start 101.545314 94.746) (end 100.384686 94.746) (width 0.2) (layer "F.Cu") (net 8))
 (segment (start 100.384686 94.746) (end 99.564 93.925314) (width 0.2) (layer "F.Cu") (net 8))
 (segment (start 139.7 108.14237) (end 132.75963 101.202) (width 0.2) (layer "F.Cu") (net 8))
 (segment (start 108.001314 101.202) (end 101.545314 94.746) (width 0.2) (layer "F.Cu") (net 8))
 (segment (start 99.564 85.856) (end 99.695 85.725) (width 0.2) (layer "F.Cu") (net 8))
 (segment (start 137.16 107.315) (end 137.16 109.22) (width 0.2) (layer "B.Cu") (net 9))
 (segment (start 115.57 85.725) (end 137.16 107.315) (width 0.2) (layer "B.Cu") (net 9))
 (segment (start 131.445 85.725) (end 138.223 92.503) (width 0.2) (layer "B.Cu") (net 2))
 (segment (start 138.223 109.66031) (end 137.39331 110.49) (width 0.2) (layer "B.Cu") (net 2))
 (segment (start 135.89 110.49) (end 134.62 109.22) (width 0.2) (layer "B.Cu") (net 2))
 (segment (start 138.223 92.503) (end 138.223 109.66031) (width 0.2) (layer "B.Cu") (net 2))
 (segment (start 137.39331 110.49) (end 135.89 110.49) (width 0.2) (layer "B.Cu") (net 2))
 (segment (start 139.95363 100.776) (end 108.396 100.776) (width 0.2) (layer "F.Cu") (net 5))
 (segment (start 147.32 108.14237) (end 139.95363 100.776) (width 0.2) (layer "F.Cu") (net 5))
 (segment (start 108.396 100.776) (end 100.965 93.345) (width 0.2) (layer "F.Cu") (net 5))
 (segment (start 147.32 109.22) (end 147.32 108.14237) (width 0.2) (layer "F.Cu") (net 5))
 (segment (start 144.78 109.22) (end 145.843 110.283) (width 0.2) (layer "F.Cu") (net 6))
 (segment (start 148.383 109.66031) (end 148.383 107.129374) (width 0.2) (layer "F.Cu") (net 6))
 (segment (start 145.843 110.283) (end 147.76031 110.283) (width 0.2) (layer "F.Cu") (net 6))
 (segment (start 147.76031 110.283) (end 148.383 109.66031) (width 0.2) (layer "F.Cu") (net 6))
 (segment (start 134.598626 93.345) (end 120.015 93.345) (width 0.2) (layer "F.Cu") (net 6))
 (segment (start 148.383 107.129374) (end 134.598626 93.345) (width 0.2) (layer "F.Cu") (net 6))
 (segment (start 100.965 112.395) (end 103.077 110.283) (width 0.2) (layer "F.Cu") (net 7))
 (segment (start 103.077 110.283) (end 141.177 110.283) (width 0.2) (layer "F.Cu") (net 7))
 (segment (start 141.177 110.283) (end 142.24 109.22) (width 0.2) (layer "F.Cu") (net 7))
 (segment (start 142.24 83.185) (end 144.78 83.185) (width 0.2) (layer "F.Cu") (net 3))
 (segment (start 144.78 83.185) (end 147.32 80.645) (width 0.2) (layer "F.Cu") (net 3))
 (segment (start 133.751 110.891) (end 132.08 109.22) (width 0.2) (layer "B.Cu") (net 10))
 (segment (start 137.55941 110.891) (end 133.751 110.891) (width 0.2) (layer "B.Cu") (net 10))
 (segment (start 138.637 94.408) (end 138.637 109.81341) (width 0.2) (layer "B.Cu") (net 10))
 (segment (start 138.637 109.81341) (end 137.55941 110.891) (width 0.2) (layer "B.Cu") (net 10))
 (segment (start 147.32 85.725) (end 138.637 94.408) (width 0.2) (layer "B.Cu") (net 10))
 (segment (start 125.095 112.395) (end 137.16 124.46) (width 0.2) (layer "F.Cu") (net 13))
 (segment (start 120.015 112.395) (end 125.095 112.395) (width 0.2) (layer "F.Cu") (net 13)))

